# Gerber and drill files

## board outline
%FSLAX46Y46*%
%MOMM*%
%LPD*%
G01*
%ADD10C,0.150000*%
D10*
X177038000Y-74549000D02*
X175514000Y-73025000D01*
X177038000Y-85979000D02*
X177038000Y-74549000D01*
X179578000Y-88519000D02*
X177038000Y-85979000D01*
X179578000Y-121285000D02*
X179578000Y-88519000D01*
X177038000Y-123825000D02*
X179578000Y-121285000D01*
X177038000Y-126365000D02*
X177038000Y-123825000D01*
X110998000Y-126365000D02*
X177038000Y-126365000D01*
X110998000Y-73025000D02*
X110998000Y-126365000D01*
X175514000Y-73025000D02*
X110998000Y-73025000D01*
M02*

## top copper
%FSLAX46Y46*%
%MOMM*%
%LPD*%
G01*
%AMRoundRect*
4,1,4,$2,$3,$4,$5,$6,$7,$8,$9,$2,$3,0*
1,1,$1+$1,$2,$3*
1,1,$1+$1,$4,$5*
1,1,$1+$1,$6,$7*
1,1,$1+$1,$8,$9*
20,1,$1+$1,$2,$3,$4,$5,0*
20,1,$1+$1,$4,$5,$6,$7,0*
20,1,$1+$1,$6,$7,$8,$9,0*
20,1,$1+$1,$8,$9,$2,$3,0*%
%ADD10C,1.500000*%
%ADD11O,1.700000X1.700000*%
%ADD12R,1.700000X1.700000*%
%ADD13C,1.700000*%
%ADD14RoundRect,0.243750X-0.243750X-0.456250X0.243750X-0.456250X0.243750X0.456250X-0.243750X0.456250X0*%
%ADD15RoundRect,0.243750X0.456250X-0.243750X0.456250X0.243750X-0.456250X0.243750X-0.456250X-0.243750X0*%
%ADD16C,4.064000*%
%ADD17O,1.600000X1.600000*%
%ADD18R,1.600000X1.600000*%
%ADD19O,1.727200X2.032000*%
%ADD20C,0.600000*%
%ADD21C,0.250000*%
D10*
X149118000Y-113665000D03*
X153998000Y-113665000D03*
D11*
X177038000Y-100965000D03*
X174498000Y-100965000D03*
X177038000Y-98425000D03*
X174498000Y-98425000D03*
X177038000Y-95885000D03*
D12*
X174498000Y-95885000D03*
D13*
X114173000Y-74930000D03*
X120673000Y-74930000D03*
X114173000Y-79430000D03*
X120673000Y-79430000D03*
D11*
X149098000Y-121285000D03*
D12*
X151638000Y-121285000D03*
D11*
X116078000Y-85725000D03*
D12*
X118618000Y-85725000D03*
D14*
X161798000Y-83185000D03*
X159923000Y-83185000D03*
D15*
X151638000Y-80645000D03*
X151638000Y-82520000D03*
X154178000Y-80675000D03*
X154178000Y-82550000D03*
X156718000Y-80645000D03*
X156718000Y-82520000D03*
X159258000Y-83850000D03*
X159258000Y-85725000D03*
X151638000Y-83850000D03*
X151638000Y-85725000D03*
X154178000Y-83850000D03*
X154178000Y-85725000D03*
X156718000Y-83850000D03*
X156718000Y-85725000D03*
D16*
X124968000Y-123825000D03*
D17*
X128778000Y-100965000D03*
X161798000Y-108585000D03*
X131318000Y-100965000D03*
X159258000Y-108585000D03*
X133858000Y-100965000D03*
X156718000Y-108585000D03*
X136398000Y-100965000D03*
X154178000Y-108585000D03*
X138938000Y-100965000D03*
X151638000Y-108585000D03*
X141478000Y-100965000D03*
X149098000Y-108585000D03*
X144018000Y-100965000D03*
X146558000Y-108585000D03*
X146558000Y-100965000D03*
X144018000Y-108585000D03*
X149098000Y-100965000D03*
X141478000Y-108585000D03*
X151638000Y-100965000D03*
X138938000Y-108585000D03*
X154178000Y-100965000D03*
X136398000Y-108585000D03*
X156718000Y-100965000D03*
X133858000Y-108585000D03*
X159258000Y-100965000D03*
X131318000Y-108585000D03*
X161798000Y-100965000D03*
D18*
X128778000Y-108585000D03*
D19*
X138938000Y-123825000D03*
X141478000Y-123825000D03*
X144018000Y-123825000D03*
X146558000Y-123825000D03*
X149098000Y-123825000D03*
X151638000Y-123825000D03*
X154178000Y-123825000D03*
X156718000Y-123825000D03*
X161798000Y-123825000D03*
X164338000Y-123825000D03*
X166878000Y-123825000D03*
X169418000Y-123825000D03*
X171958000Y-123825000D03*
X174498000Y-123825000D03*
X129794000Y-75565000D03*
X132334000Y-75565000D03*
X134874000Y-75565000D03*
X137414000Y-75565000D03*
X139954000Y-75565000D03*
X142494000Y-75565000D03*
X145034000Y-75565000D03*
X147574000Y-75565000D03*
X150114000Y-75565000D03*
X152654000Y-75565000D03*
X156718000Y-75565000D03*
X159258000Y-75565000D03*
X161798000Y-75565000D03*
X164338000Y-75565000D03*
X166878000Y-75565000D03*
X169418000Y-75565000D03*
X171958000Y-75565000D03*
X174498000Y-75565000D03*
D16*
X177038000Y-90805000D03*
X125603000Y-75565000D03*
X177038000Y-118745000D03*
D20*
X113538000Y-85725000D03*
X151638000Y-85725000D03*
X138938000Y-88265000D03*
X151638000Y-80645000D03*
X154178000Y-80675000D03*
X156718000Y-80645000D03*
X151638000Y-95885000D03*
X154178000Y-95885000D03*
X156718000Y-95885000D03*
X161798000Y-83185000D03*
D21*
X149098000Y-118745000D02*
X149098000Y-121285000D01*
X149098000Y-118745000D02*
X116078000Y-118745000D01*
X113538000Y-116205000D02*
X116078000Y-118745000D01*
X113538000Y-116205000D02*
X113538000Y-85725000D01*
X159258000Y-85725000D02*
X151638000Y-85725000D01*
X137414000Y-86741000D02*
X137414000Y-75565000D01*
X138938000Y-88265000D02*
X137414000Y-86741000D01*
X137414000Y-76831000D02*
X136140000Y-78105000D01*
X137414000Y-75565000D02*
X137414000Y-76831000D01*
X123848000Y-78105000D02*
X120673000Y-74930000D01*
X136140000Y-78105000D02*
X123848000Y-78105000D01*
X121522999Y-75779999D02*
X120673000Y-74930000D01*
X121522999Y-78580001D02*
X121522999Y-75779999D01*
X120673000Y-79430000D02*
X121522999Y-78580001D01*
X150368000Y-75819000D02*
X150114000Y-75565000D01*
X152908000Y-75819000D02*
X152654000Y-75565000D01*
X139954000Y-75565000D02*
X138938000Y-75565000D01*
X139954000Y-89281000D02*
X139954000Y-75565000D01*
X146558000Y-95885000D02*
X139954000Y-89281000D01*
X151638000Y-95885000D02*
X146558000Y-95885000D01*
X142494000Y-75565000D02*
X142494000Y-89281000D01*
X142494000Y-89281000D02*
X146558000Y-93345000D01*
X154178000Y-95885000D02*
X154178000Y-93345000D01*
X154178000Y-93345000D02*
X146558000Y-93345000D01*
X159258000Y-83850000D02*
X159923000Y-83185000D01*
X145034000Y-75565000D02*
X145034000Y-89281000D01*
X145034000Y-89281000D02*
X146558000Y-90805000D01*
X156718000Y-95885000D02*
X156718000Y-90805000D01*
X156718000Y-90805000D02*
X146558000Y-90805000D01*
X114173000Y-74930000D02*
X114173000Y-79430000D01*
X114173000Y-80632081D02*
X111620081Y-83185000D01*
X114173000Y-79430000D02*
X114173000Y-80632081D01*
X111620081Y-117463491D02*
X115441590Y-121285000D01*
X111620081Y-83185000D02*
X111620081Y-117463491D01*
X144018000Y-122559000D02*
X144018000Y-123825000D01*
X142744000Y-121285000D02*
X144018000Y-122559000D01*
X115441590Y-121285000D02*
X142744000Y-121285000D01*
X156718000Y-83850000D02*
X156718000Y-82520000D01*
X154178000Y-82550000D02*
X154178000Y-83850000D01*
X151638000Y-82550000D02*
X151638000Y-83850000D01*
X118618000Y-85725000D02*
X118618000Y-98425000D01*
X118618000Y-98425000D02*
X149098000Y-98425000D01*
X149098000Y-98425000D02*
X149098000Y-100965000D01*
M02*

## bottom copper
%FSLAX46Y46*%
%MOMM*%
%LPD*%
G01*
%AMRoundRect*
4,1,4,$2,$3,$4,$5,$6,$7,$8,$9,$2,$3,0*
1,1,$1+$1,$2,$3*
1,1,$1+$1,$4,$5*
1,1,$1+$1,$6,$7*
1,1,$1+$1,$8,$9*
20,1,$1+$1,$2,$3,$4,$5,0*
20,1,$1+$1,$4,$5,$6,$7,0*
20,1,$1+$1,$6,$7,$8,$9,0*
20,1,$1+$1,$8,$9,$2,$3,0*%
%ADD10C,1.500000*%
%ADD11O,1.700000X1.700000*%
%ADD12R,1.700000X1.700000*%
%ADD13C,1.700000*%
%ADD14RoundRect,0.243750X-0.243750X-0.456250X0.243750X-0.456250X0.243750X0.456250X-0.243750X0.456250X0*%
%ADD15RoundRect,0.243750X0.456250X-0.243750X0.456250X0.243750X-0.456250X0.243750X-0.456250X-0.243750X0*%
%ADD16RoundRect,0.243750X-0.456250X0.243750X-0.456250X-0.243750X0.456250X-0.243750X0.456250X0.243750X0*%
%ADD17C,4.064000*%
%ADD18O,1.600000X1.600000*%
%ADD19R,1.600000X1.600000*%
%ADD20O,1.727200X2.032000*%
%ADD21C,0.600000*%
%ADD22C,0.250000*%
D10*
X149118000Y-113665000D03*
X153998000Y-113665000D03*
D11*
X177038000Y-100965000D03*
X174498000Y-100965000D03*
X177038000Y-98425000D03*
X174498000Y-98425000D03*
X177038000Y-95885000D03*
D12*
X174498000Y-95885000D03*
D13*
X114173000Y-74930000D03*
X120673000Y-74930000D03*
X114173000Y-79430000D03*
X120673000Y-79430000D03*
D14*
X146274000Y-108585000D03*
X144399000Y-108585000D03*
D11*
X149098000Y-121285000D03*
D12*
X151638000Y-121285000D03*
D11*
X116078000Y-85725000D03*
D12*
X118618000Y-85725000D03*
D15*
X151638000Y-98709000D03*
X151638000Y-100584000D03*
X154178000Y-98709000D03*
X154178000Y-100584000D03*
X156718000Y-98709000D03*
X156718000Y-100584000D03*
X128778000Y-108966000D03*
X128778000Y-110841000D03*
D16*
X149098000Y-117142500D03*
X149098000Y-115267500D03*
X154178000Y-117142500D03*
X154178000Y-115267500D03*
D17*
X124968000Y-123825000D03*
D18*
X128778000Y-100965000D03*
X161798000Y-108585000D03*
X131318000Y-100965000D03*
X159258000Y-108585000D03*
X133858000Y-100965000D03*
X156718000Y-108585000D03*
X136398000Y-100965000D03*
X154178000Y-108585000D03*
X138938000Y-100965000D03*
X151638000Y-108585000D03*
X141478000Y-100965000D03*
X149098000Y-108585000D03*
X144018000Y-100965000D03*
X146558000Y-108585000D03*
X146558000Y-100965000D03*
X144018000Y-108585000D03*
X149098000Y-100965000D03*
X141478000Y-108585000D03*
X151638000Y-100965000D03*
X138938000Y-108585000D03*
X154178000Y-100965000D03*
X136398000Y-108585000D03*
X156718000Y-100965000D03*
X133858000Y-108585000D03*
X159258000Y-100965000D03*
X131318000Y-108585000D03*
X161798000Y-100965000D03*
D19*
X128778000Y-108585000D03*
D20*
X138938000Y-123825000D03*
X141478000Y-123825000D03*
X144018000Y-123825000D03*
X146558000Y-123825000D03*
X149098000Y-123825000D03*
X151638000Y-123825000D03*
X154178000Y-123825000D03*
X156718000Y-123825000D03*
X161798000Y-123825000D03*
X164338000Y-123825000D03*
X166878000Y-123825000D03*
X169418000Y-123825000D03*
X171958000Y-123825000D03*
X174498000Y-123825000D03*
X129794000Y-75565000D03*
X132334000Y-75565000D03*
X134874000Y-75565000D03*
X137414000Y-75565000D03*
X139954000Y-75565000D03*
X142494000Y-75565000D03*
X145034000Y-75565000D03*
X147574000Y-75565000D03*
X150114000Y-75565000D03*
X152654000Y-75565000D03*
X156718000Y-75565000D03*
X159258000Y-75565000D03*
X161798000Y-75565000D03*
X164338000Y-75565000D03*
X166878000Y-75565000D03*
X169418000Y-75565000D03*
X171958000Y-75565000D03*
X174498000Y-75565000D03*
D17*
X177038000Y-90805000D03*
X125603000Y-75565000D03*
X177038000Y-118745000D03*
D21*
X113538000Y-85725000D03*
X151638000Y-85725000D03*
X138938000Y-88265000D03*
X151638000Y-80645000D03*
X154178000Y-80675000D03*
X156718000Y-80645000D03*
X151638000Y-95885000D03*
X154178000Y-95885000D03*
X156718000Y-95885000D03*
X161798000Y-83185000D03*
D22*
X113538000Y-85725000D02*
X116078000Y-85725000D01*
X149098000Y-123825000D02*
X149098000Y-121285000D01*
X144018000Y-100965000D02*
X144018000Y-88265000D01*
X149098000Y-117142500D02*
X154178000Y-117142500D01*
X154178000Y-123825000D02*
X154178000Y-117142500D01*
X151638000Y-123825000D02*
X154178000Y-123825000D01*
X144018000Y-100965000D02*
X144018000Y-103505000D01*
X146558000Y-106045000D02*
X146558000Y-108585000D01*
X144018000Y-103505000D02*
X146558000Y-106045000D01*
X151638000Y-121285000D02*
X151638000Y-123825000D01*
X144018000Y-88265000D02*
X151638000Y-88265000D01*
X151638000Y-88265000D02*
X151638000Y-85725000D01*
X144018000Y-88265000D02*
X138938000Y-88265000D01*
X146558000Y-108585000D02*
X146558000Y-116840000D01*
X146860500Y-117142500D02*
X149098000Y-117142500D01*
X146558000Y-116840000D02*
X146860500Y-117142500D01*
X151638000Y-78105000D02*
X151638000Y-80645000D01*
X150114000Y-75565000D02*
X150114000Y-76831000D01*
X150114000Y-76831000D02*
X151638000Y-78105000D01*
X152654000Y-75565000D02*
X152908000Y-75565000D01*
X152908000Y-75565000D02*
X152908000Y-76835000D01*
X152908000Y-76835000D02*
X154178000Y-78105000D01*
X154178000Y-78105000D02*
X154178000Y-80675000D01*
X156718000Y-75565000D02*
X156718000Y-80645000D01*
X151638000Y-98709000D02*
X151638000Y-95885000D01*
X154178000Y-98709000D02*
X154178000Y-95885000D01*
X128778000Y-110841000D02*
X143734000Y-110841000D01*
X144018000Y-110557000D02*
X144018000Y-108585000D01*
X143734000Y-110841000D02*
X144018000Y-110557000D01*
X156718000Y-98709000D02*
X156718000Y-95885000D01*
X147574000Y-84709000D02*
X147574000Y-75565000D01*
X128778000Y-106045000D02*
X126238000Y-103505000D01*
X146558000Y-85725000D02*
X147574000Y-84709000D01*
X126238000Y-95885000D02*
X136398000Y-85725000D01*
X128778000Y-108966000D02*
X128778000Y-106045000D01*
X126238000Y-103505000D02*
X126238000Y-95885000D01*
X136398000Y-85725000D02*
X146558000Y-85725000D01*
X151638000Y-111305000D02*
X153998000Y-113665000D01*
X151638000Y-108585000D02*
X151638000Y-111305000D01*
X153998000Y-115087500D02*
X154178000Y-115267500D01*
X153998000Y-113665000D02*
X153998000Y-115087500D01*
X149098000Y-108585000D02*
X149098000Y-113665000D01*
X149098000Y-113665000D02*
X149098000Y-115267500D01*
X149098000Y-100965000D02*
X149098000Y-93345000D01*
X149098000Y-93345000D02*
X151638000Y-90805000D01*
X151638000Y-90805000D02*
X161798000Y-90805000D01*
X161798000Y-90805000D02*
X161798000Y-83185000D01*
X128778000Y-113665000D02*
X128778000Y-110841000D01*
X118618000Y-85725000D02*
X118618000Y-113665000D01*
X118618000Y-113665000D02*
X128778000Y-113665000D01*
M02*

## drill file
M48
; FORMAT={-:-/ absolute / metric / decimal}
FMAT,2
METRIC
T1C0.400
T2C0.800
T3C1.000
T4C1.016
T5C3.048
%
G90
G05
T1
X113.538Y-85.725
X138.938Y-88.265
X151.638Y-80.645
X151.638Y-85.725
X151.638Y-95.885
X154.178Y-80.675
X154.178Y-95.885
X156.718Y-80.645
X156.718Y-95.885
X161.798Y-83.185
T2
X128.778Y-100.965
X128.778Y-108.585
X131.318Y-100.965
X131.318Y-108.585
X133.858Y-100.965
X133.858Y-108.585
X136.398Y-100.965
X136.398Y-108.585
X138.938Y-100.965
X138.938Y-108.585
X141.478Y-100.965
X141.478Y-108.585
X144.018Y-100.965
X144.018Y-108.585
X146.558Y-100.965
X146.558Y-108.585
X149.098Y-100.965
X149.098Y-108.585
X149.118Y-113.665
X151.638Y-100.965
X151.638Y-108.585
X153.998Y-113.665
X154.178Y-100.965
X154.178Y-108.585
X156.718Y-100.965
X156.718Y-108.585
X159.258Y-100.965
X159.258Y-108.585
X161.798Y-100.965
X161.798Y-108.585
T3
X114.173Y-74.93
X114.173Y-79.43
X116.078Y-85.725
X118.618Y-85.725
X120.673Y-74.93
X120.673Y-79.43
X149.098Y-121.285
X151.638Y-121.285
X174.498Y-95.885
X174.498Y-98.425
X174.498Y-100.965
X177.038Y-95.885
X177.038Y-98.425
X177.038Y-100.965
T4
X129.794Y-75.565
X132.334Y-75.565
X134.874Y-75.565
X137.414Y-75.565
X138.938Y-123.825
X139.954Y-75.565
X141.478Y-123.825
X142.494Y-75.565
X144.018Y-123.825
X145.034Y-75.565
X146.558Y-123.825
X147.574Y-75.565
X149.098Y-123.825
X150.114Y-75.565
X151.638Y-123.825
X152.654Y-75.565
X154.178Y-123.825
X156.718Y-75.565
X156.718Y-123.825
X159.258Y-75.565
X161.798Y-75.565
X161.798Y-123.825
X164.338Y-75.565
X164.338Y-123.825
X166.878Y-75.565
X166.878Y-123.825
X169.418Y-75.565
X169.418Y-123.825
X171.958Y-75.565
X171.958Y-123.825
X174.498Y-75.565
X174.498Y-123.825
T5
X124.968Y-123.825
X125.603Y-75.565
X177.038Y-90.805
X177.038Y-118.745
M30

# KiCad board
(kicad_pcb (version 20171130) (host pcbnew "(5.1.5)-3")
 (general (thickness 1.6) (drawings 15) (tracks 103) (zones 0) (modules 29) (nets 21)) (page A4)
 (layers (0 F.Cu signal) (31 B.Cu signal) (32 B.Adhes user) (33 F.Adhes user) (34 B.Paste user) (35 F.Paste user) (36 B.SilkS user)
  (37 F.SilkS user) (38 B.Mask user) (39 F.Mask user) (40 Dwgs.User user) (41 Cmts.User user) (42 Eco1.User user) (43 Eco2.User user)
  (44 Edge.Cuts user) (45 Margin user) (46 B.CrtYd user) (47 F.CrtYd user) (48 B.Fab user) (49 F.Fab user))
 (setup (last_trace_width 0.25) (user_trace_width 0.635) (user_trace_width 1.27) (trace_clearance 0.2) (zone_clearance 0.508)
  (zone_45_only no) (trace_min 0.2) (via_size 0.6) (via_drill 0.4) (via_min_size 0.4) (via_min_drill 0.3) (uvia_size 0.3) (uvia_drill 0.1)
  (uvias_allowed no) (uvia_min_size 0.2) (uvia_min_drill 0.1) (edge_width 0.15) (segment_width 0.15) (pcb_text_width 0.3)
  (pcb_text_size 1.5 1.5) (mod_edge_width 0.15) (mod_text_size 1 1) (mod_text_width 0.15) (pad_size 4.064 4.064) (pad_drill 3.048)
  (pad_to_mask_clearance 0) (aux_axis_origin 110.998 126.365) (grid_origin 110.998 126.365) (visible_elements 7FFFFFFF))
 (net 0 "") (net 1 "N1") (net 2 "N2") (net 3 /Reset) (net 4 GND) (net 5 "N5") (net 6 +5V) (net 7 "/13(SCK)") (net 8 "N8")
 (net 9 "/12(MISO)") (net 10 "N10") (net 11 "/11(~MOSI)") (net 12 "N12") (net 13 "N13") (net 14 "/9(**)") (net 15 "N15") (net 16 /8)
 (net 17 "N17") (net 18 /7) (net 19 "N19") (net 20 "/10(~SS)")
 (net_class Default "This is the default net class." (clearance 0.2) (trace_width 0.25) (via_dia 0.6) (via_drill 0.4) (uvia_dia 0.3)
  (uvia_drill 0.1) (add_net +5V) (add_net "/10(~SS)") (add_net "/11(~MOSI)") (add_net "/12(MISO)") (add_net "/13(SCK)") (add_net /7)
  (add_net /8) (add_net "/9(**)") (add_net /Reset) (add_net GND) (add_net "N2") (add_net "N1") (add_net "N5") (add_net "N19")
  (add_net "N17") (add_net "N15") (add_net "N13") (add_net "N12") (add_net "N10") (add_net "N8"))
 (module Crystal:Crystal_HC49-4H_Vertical (layer F.Cu) (at 153.998 113.665 180)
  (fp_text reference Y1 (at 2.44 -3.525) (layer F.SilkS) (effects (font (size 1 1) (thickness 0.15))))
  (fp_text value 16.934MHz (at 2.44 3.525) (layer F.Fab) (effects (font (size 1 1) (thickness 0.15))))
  (pad 2 thru_hole circle (at 4.88 0 180) (size 1.5 1.5) (drill 0.8) (layers *.Cu *.Mask) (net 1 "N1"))
  (pad 1 thru_hole circle (at 0 0 180) (size 1.5 1.5) (drill 0.8) (layers *.Cu *.Mask) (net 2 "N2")))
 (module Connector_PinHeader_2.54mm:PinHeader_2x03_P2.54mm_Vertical (layer F.Cu) (at 174.498 95.885)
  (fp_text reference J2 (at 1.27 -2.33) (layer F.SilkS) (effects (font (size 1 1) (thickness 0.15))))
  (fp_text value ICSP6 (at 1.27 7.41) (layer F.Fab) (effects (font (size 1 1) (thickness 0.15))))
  (pad 6 thru_hole oval (at 2.54 5.08) (size 1.7 1.7) (drill 1) (layers *.Cu *.Mask))
  (pad 5 thru_hole oval (at 0 5.08) (size 1.7 1.7) (drill 1) (layers *.Cu *.Mask))
  (pad 4 thru_hole oval (at 2.54 2.54) (size 1.7 1.7) (drill 1) (layers *.Cu *.Mask))
  (pad 3 thru_hole oval (at 0 2.54) (size 1.7 1.7) (drill 1) (layers *.Cu *.Mask))
  (pad 2 thru_hole oval (at 2.54 0) (size 1.7 1.7) (drill 1) (layers *.Cu *.Mask))
  (pad 1 thru_hole rect (at 0 0) (size 1.7 1.7) (drill 1) (layers *.Cu *.Mask)))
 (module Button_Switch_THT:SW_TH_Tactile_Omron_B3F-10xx (layer F.Cu) (at 114.173 74.93)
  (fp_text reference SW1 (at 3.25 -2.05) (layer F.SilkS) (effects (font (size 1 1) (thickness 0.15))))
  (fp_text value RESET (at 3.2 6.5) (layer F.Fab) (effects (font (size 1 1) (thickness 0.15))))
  (pad 1 thru_hole circle (at 0 0) (size 1.7 1.7) (drill 1) (layers *.Cu *.Mask) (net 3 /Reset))
  (pad 2 thru_hole circle (at 6.5 0) (size 1.7 1.7) (drill 1) (layers *.Cu *.Mask) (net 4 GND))
  (pad 3 thru_hole circle (at 0 4.5) (size 1.7 1.7) (drill 1) (layers *.Cu *.Mask) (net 3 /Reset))
  (pad 4 thru_hole circle (at 6.5 4.5) (size 1.7 1.7) (drill 1) (layers *.Cu *.Mask) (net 4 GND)))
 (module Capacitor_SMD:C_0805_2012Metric (layer B.Cu) (at 145.3365 108.585)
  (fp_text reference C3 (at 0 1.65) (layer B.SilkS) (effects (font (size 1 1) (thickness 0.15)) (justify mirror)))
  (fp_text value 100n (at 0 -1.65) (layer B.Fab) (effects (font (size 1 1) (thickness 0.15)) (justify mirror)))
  (pad 2 smd roundrect (at 0.9375 0) (size 0.975 1.4) (layers B.Cu B.Paste B.Mask) (roundrect_rratio 0.25) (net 4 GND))
  (pad 1 smd roundrect (at -0.9375 0) (size 0.975 1.4) (layers B.Cu B.Paste B.Mask) (roundrect_rratio 0.25) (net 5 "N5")))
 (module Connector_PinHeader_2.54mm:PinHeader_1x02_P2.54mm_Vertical (layer F.Cu) (at 151.638 121.285 270)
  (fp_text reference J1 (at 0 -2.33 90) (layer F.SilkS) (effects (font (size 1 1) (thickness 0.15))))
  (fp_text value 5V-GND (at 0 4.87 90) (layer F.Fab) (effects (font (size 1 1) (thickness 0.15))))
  (pad 2 thru_hole oval (at 0 2.54 270) (size 1.7 1.7) (drill 1) (layers *.Cu *.Mask) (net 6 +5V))
  (pad 1 thru_hole rect (at 0 0 270) (size 1.7 1.7) (drill 1) (layers *.Cu *.Mask) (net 4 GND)))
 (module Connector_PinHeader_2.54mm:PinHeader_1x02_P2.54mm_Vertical (layer F.Cu) (at 118.618 85.725 270)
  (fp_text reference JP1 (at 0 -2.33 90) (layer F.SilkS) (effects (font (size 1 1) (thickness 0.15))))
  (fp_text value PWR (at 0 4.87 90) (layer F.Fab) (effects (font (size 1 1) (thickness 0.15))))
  (pad 2 thru_hole oval (at 0 2.54 270) (size 1.7 1.7) (drill 1) (layers *.Cu *.Mask) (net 6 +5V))
  (pad 1 thru_hole rect (at 0 0 270) (size 1.7 1.7) (drill 1) (layers *.Cu *.Mask) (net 5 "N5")))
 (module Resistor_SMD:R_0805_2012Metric (layer B.Cu) (at 151.638 99.6465 90)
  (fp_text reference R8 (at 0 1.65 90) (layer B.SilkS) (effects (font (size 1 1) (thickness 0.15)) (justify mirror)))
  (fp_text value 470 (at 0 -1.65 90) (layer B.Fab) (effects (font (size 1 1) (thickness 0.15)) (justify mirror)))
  (pad 2 smd roundrect (at 0.9375 0 90) (size 0.975 1.4) (layers B.Cu B.Paste B.Mask) (roundrect_rratio 0.25) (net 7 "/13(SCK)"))
  (pad 1 smd roundrect (at -0.9375 0 90) (size 0.975 1.4) (layers B.Cu B.Paste B.Mask) (roundrect_rratio 0.25) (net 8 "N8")))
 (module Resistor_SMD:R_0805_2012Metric (layer B.Cu) (at 154.178 99.6465 90)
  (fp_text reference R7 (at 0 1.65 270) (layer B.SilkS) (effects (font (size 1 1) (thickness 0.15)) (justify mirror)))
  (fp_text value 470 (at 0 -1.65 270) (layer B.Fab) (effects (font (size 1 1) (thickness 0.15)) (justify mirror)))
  (pad 2 smd roundrect (at 0.9375 0 90) (size 0.975 1.4) (layers B.Cu B.Paste B.Mask) (roundrect_rratio 0.25) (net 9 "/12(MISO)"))
  (pad 1 smd roundrect (at -0.9375 0 90) (size 0.975 1.4) (layers B.Cu B.Paste B.Mask) (roundrect_rratio 0.25) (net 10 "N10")))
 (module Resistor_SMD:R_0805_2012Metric (layer B.Cu) (at 156.718 99.6465 90)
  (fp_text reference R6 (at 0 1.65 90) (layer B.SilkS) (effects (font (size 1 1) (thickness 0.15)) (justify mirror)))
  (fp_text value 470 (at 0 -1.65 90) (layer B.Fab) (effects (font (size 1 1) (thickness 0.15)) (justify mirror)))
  (pad 2 smd roundrect (at 0.9375 0 90) (size 0.975 1.4) (layers B.Cu B.Paste B.Mask) (roundrect_rratio 0.25) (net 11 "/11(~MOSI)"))
  (pad 1 smd roundrect (at -0.9375 0 90) (size 0.975 1.4) (layers B.Cu B.Paste B.Mask) (roundrect_rratio 0.25) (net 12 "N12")))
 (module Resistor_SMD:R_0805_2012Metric (layer F.Cu) (at 160.8605 83.185)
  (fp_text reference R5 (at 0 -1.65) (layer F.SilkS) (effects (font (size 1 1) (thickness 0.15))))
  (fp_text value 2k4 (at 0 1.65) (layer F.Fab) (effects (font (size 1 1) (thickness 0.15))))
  (pad 2 smd roundrect (at 0.9375 0) (size 0.975 1.4) (layers F.Cu F.Paste F.Mask) (roundrect_rratio 0.25) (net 5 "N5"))
  (pad 1 smd roundrect (at -0.9375 0) (size 0.975 1.4) (layers F.Cu F.Paste F.Mask) (roundrect_rratio 0.25) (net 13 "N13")))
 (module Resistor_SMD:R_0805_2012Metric (layer F.Cu) (at 151.638 81.5825 90)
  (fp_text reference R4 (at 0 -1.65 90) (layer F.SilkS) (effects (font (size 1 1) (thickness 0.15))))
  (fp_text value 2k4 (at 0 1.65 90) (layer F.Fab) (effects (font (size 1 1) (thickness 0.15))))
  (pad 2 smd roundrect (at 0.9375 0 90) (size 0.975 1.4) (layers F.Cu F.Paste F.Mask) (roundrect_rratio 0.25) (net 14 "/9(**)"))
  (pad 1 smd roundrect (at -0.9375 0 90) (size 0.975 1.4) (layers F.Cu F.Paste F.Mask) (roundrect_rratio 0.25) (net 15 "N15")))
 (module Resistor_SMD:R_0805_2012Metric (layer F.Cu) (at 154.178 81.6125 90)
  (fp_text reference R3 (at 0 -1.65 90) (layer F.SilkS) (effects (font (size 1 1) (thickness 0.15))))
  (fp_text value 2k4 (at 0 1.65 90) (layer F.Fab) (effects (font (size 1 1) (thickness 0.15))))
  (pad 2 smd roundrect (at 0.9375 0 90) (size 0.975 1.4) (layers F.Cu F.Paste F.Mask) (roundrect_rratio 0.25) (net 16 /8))
  (pad 1 smd roundrect (at -0.9375 0 90) (size 0.975 1.4) (layers F.Cu F.Paste F.Mask) (roundrect_rratio 0.25) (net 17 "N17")))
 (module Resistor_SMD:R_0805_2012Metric (layer F.Cu) (at 156.718 81.5825 90)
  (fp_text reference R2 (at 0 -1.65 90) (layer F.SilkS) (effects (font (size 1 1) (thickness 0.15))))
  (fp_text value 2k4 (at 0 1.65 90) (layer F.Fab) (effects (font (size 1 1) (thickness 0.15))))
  (pad 2 smd roundrect (at 0.9375 0 90) (size 0.975 1.4) (layers F.Cu F.Paste F.Mask) (roundrect_rratio 0.25) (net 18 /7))
  (pad 1 smd roundrect (at -0.9375 0 90) (size 0.975 1.4) (layers F.Cu F.Paste F.Mask) (roundrect_rratio 0.25) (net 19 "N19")))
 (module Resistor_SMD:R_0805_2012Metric (layer B.Cu) (at 128.778 109.9035 90)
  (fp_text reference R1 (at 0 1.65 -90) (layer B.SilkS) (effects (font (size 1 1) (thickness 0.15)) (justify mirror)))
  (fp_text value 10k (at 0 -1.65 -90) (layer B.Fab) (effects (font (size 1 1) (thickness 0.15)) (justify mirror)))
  (pad 2 smd roundrect (at 0.9375 0 90) (size 0.975 1.4) (layers B.Cu B.Paste B.Mask) (roundrect_rratio 0.25) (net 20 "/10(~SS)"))
  (pad 1 smd roundrect (at -0.9375 0 90) (size 0.975 1.4) (layers B.Cu B.Paste B.Mask) (roundrect_rratio 0.25) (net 5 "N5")))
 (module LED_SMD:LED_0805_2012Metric (layer F.Cu) (at 159.258 84.7875 90)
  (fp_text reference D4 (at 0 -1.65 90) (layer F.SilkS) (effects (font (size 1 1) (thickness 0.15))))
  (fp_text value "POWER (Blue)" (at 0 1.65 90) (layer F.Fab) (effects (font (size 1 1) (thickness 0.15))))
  (pad 2 smd roundrect (at 0.9375 0 90) (size 0.975 1.4) (layers F.Cu F.Paste F.Mask) (roundrect_rratio 0.25) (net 13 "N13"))
  (pad 1 smd roundrect (at -0.9375 0 90) (size 0.975 1.4) (layers F.Cu F.Paste F.Mask) (roundrect_rratio 0.25) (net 4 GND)))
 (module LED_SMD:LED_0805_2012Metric (layer F.Cu) (at 151.638 84.7875 90)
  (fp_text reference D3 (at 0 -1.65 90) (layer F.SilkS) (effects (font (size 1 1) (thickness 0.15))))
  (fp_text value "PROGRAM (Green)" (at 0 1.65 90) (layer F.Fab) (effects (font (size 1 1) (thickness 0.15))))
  (pad 2 smd roundrect (at 0.9375 0 90) (size 0.975 1.4) (layers F.Cu F.Paste F.Mask) (roundrect_rratio 0.25) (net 15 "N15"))
  (pad 1 smd roundrect (at -0.9375 0 90) (size 0.975 1.4) (layers F.Cu F.Paste F.Mask) (roundrect_rratio 0.25) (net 4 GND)))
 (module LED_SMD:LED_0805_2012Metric (layer F.Cu) (at 154.178 84.7875 90)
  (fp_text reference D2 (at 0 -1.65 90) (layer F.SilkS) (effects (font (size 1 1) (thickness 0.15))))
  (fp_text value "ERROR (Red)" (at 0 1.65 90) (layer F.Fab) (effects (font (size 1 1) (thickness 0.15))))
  (pad 2 smd roundrect (at 0.9375 0 90) (size 0.975 1.4) (layers F.Cu F.Paste F.Mask) (roundrect_rratio 0.25) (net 17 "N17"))
  (pad 1 smd roundrect (at -0.9375 0 90) (size 0.975 1.4) (layers F.Cu F.Paste F.Mask) (roundrect_rratio 0.25) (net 4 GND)))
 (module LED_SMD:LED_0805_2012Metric (layer F.Cu) (at 156.718 84.7875 90)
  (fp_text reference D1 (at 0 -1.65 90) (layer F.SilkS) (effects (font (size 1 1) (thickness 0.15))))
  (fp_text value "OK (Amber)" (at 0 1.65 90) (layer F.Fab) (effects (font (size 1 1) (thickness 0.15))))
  (pad 2 smd roundrect (at 0.9375 0 90) (size 0.975 1.4) (layers F.Cu F.Paste F.Mask) (roundrect_rratio 0.25) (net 19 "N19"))
  (pad 1 smd roundrect (at -0.9375 0 90) (size 0.975 1.4) (layers F.Cu F.Paste F.Mask) (roundrect_rratio 0.25) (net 4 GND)))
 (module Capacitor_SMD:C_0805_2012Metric (layer B.Cu) (at 149.098 116.205 270)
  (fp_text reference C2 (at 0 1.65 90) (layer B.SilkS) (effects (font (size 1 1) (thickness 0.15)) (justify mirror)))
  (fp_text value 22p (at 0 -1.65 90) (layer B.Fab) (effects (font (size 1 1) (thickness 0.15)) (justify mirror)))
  (pad 2 smd roundrect (at 0.9375 0 270) (size 0.975 1.4) (layers B.Cu B.Paste B.Mask) (roundrect_rratio 0.25) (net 4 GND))
  (pad 1 smd roundrect (at -0.9375 0 270) (size 0.975 1.4) (layers B.Cu B.Paste B.Mask) (roundrect_rratio 0.25) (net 1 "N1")))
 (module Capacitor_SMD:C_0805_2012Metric (layer B.Cu) (at 154.178 116.205 270)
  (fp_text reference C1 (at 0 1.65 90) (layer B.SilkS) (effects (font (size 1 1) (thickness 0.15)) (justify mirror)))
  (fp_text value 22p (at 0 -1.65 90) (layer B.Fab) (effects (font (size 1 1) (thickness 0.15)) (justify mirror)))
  (pad 2 smd roundrect (at 0.9375 0 270) (size 0.975 1.4) (layers B.Cu B.Paste B.Mask) (roundrect_rratio 0.25) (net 4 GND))
  (pad 1 smd roundrect (at -0.9375 0 270) (size 0.975 1.4) (layers B.Cu B.Paste B.Mask) (roundrect_rratio 0.25) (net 2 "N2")))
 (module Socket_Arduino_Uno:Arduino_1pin (layer F.Cu) (at 124.968 123.825 90)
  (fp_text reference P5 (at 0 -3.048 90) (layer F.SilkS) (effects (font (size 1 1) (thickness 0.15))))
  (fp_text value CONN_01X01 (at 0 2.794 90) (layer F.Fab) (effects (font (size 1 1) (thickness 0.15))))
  (pad 1 thru_hole circle (at 0 0 90) (size 4.064 4.064) (drill 3.048) (layers *.Cu *.Mask F.SilkS)))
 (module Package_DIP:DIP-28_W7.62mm (layer F.Cu) (at 128.778 108.585 90)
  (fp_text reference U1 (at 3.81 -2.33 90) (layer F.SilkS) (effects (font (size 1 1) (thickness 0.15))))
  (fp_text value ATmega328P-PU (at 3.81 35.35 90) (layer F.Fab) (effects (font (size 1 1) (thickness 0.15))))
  (pad 28 thru_hole oval (at 7.62 0 90) (size 1.6 1.6) (drill 0.8) (layers *.Cu *.Mask))
  (pad 14 thru_hole oval (at 0 33.02 90) (size 1.6 1.6) (drill 0.8) (layers *.Cu *.Mask))
  (pad 27 thru_hole oval (at 7.62 2.54 90) (size 1.6 1.6) (drill 0.8) (layers *.Cu *.Mask))
  (pad 13 thru_hole oval (at 0 30.48 90) (size 1.6 1.6) (drill 0.8) (layers *.Cu *.Mask))
  (pad 26 thru_hole oval (at 7.62 5.08 90) (size 1.6 1.6) (drill 0.8) (layers *.Cu *.Mask))
  (pad 12 thru_hole oval (at 0 27.94 90) (size 1.6 1.6) (drill 0.8) (layers *.Cu *.Mask))
  (pad 25 thru_hole oval (at 7.62 7.62 90) (size 1.6 1.6) (drill 0.8) (layers *.Cu *.Mask))
  (pad 11 thru_hole oval (at 0 25.4 90) (size 1.6 1.6) (drill 0.8) (layers *.Cu *.Mask))
  (pad 24 thru_hole oval (at 7.62 10.16 90) (size 1.6 1.6) (drill 0.8) (layers *.Cu *.Mask))
  (pad 10 thru_hole oval (at 0 22.86 90) (size 1.6 1.6) (drill 0.8) (layers *.Cu *.Mask) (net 2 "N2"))
  (pad 23 thru_hole oval (at 7.62 12.7 90) (size 1.6 1.6) (drill 0.8) (layers *.Cu *.Mask))
  (pad 9 thru_hole oval (at 0 20.32 90) (size 1.6 1.6) (drill 0.8) (layers *.Cu *.Mask) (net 1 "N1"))
  (pad 22 thru_hole oval (at 7.62 15.24 90) (size 1.6 1.6) (drill 0.8) (layers *.Cu *.Mask) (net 4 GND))
  (pad 8 thru_hole oval (at 0 17.78 90) (size 1.6 1.6) (drill 0.8) (layers *.Cu *.Mask) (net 4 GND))
  (pad 21 thru_hole oval (at 7.62 17.78 90) (size 1.6 1.6) (drill 0.8) (layers *.Cu *.Mask))
  (pad 7 thru_hole oval (at 0 15.24 90) (size 1.6 1.6) (drill 0.8) (layers *.Cu *.Mask) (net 5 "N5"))
  (pad 20 thru_hole oval (at 7.62 20.32 90) (size 1.6 1.6) (drill 0.8) (layers *.Cu *.Mask) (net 5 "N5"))
  (pad 6 thru_hole oval (at 0 12.7 90) (size 1.6 1.6) (drill 0.8) (layers *.Cu *.Mask))
  (pad 19 thru_hole oval (at 7.62 22.86 90) (size 1.6 1.6) (drill 0.8) (layers *.Cu *.Mask) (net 8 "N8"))
  (pad 5 thru_hole oval (at 0 10.16 90) (size 1.6 1.6) (drill 0.8) (layers *.Cu *.Mask))
  (pad 18 thru_hole oval (at 7.62 25.4 90) (size 1.6 1.6) (drill 0.8) (layers *.Cu *.Mask) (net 10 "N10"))
  (pad 4 thru_hole oval (at 0 7.62 90) (size 1.6 1.6) (drill 0.8) (layers *.Cu *.Mask))
  (pad 17 thru_hole oval (at 7.62 27.94 90) (size 1.6 1.6) (drill 0.8) (layers *.Cu *.Mask) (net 12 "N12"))
  (pad 3 thru_hole oval (at 0 5.08 90) (size 1.6 1.6) (drill 0.8) (layers *.Cu *.Mask))
  (pad 16 thru_hole oval (at 7.62 30.48 90) (size 1.6 1.6) (drill 0.8) (layers *.Cu *.Mask))
  (pad 2 thru_hole oval (at 0 2.54 90) (size 1.6 1.6) (drill 0.8) (layers *.Cu *.Mask))
  (pad 15 thru_hole oval (at 7.62 33.02 90) (size 1.6 1.6) (drill 0.8) (layers *.Cu *.Mask))
  (pad 1 thru_hole rect (at 0 0 90) (size 1.6 1.6) (drill 0.8) (layers *.Cu *.Mask) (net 20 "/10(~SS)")))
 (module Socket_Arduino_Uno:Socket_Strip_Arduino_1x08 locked (layer F.Cu) (at 138.938 123.825)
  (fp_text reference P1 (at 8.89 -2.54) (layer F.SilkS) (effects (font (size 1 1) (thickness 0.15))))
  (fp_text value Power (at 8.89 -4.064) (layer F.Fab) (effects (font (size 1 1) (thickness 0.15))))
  (pad 1 thru_hole oval (at 0 0) (size 1.7272 2.032) (drill 1.016) (layers *.Cu *.Mask F.SilkS))
  (pad 2 thru_hole oval (at 2.54 0) (size 1.7272 2.032) (drill 1.016) (layers *.Cu *.Mask F.SilkS))
  (pad 3 thru_hole oval (at 5.08 0) (size 1.7272 2.032) (drill 1.016) (layers *.Cu *.Mask F.SilkS) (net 3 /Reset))
  (pad 4 thru_hole oval (at 7.62 0) (size 1.7272 2.032) (drill 1.016) (layers *.Cu *.Mask F.SilkS))
  (pad 5 thru_hole oval (at 10.16 0) (size 1.7272 2.032) (drill 1.016) (layers *.Cu *.Mask F.SilkS) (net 6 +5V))
  (pad 6 thru_hole oval (at 12.7 0) (size 1.7272 2.032) (drill 1.016) (layers *.Cu *.Mask F.SilkS) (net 4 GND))
  (pad 7 thru_hole oval (at 15.24 0) (size 1.7272 2.032) (drill 1.016) (layers *.Cu *.Mask F.SilkS) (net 4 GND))
  (pad 8 thru_hole oval (at 17.78 0) (size 1.7272 2.032) (drill 1.016) (layers *.Cu *.Mask F.SilkS)))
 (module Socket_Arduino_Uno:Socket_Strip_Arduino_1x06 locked (layer F.Cu) (at 161.798 123.825)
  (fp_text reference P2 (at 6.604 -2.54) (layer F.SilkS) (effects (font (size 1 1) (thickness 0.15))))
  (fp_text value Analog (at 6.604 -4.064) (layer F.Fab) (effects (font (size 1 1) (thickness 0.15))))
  (pad 1 thru_hole oval (at 0 0) (size 1.7272 2.032) (drill 1.016) (layers *.Cu *.Mask F.SilkS))
  (pad 2 thru_hole oval (at 2.54 0) (size 1.7272 2.032) (drill 1.016) (layers *.Cu *.Mask F.SilkS))
  (pad 3 thru_hole oval (at 5.08 0) (size 1.7272 2.032) (drill 1.016) (layers *.Cu *.Mask F.SilkS))
  (pad 4 thru_hole oval (at 7.62 0) (size 1.7272 2.032) (drill 1.016) (layers *.Cu *.Mask F.SilkS))
  (pad 5 thru_hole oval (at 10.16 0) (size 1.7272 2.032) (drill 1.016) (layers *.Cu *.Mask F.SilkS))
  (pad 6 thru_hole oval (at 12.7 0) (size 1.7272 2.032) (drill 1.016) (layers *.Cu *.Mask F.SilkS)))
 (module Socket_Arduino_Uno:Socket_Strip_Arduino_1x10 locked (layer F.Cu) (at 129.794 75.565)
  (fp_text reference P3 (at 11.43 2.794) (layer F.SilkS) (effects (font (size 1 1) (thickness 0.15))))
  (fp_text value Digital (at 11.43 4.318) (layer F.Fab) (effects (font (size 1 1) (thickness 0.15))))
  (pad 1 thru_hole oval (at 0 0) (size 1.7272 2.032) (drill 1.016) (layers *.Cu *.Mask F.SilkS))
  (pad 2 thru_hole oval (at 2.54 0) (size 1.7272 2.032) (drill 1.016) (layers *.Cu *.Mask F.SilkS))
  (pad 3 thru_hole oval (at 5.08 0) (size 1.7272 2.032) (drill 1.016) (layers *.Cu *.Mask F.SilkS))
  (pad 4 thru_hole oval (at 7.62 0) (size 1.7272 2.032) (drill 1.016) (layers *.Cu *.Mask F.SilkS) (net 4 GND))
  (pad 5 thru_hole oval (at 10.16 0) (size 1.7272 2.032) (drill 1.016) (layers *.Cu *.Mask F.SilkS) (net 7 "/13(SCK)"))
  (pad 6 thru_hole oval (at 12.7 0) (size 1.7272 2.032) (drill 1.016) (layers *.Cu *.Mask F.SilkS) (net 9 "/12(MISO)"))
  (pad 7 thru_hole oval (at 15.24 0) (size 1.7272 2.032) (drill 1.016) (layers *.Cu *.Mask F.SilkS) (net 11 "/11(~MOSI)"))
  (pad 8 thru_hole oval (at 17.78 0) (size 1.7272 2.032) (drill 1.016) (layers *.Cu *.Mask F.SilkS) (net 20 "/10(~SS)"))
  (pad 9 thru_hole oval (at 20.32 0) (size 1.7272 2.032) (drill 1.016) (layers *.Cu *.Mask F.SilkS) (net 14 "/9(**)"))
  (pad 10 thru_hole oval (at 22.86 0) (size 1.7272 2.032) (drill 1.016) (layers *.Cu *.Mask F.SilkS) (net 16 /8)))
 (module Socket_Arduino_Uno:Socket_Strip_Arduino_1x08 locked (layer F.Cu) (at 156.718 75.565)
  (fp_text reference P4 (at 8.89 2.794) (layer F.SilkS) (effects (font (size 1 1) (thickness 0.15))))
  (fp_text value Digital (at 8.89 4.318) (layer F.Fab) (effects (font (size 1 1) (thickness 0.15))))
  (pad 1 thru_hole oval (at 0 0) (size 1.7272 2.032) (drill 1.016) (layers *.Cu *.Mask F.SilkS) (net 18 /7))
  (pad 2 thru_hole oval (at 2.54 0) (size 1.7272 2.032) (drill 1.016) (layers *.Cu *.Mask F.SilkS))
  (pad 3 thru_hole oval (at 5.08 0) (size 1.7272 2.032) (drill 1.016) (layers *.Cu *.Mask F.SilkS))
  (pad 4 thru_hole oval (at 7.62 0) (size 1.7272 2.032) (drill 1.016) (layers *.Cu *.Mask F.SilkS))
  (pad 5 thru_hole oval (at 10.16 0) (size 1.7272 2.032) (drill 1.016) (layers *.Cu *.Mask F.SilkS))
  (pad 6 thru_hole oval (at 12.7 0) (size 1.7272 2.032) (drill 1.016) (layers *.Cu *.Mask F.SilkS))
  (pad 7 thru_hole oval (at 15.24 0) (size 1.7272 2.032) (drill 1.016) (layers *.Cu *.Mask F.SilkS))
  (pad 8 thru_hole oval (at 17.78 0) (size 1.7272 2.032) (drill 1.016) (layers *.Cu *.Mask F.SilkS)))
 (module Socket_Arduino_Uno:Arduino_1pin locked (layer F.Cu) (at 177.038 90.805 90)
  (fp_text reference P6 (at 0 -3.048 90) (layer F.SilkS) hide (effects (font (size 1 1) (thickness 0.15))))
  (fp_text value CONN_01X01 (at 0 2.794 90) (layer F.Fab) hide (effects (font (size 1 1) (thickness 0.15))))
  (pad 1 thru_hole circle (at 0 0 90) (size 4.064 4.064) (drill 3.048) (layers *.Cu *.Mask F.SilkS)))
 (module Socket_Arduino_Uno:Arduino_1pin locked (layer F.Cu) (at 125.603 75.565 90)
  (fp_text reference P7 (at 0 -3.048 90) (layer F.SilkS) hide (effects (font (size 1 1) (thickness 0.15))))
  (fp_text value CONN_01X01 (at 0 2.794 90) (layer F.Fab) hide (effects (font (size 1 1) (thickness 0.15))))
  (pad 1 thru_hole circle (at 0 0 90) (size 4.064 4.064) (drill 3.048) (layers *.Cu *.Mask F.SilkS)))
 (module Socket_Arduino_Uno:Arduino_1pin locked (layer F.Cu) (at 177.038 118.745 90)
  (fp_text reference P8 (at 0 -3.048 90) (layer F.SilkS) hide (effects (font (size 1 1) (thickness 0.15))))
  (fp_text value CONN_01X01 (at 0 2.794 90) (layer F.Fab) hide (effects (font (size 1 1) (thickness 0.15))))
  (pad 1 thru_hole circle (at 0 0 90) (size 4.064 4.064) (drill 3.048) (layers *.Cu *.Mask F.SilkS)))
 (gr_line (start 177.038 74.549) (end 175.514 73.025) (angle 90) (layer Edge.Cuts) (width 0.15))
 (gr_line (start 177.038 85.979) (end 177.038 74.549) (angle 90) (layer Edge.Cuts) (width 0.15))
 (gr_line (start 179.578 88.519) (end 177.038 85.979) (angle 90) (layer Edge.Cuts) (width 0.15))
 (gr_line (start 179.578 121.285) (end 179.578 88.519) (angle 90) (layer Edge.Cuts) (width 0.15))
 (gr_line (start 177.038 123.825) (end 179.578 121.285) (angle 90) (layer Edge.Cuts) (width 0.15))
 (gr_line (start 177.038 126.365) (end 177.038 123.825) (angle 90) (layer Edge.Cuts) (width 0.15))
 (gr_line (start 110.998 126.365) (end 177.038 126.365) (angle 90) (layer Edge.Cuts) (width 0.15))
 (gr_line (start 110.998 73.025) (end 110.998 126.365) (angle 90) (layer Edge.Cuts) (width 0.15))
 (gr_line (start 175.514 73.025) (end 110.998 73.025) (angle 90) (layer Edge.Cuts) (width 0.15))
 (via (at 113.538 85.725) (size 0.6) (drill 0.4) (layers F.Cu B.Cu) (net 6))
 (segment (start 113.538 85.725) (end 116.078 85.725) (width 0.25) (layer B.Cu) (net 6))
 (segment (start 149.098 123.825) (end 149.098 121.285) (width 0.25) (layer B.Cu) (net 6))
 (segment (start 149.098 118.745) (end 149.098 121.285) (width 0.25) (layer F.Cu) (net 6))
 (segment (start 149.098 118.745) (end 116.078 118.745) (width 0.25) (layer F.Cu) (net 6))
 (segment (start 113.538 116.205) (end 116.078 118.745) (width 0.25) (layer F.Cu) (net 6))
 (segment (start 113.538 116.205) (end 113.538 85.725) (width 0.25) (layer F.Cu) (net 6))
 (segment (start 144.018 100.965) (end 144.018 88.265) (width 0.25) (layer B.Cu) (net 4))
 (segment (start 149.098 117.1425) (end 154.178 117.1425) (width 0.25) (layer B.Cu) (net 4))
 (segment (start 154.178 123.825) (end 154.178 117.1425) (width 0.25) (layer B.Cu) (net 4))
 (segment (start 151.638 123.825) (end 154.178 123.825) (width 0.25) (layer B.Cu) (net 4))
 (segment (start 144.018 100.965) (end 144.018 103.505) (width 0.25) (layer B.Cu) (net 4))
 (segment (start 146.558 106.045) (end 146.558 108.585) (width 0.25) (layer B.Cu) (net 4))
 (segment (start 144.018 103.505) (end 146.558 106.045) (width 0.25) (layer B.Cu) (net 4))
 (segment (start 151.638 121.285) (end 151.638 123.825) (width 0.25) (layer B.Cu) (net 4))
 (segment (start 159.258 85.725) (end 151.638 85.725) (width 0.25) (layer F.Cu) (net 4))
 (segment (start 144.018 88.265) (end 151.638 88.265) (width 0.25) (layer B.Cu) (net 4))
 (segment (start 151.638 88.265) (end 151.638 85.725) (width 0.25) (layer B.Cu) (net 4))
 (via (at 151.638 85.725) (size 0.6) (drill 0.4) (layers F.Cu B.Cu) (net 4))
 (segment (start 144.018 88.265) (end 138.938 88.265) (width 0.25) (layer B.Cu) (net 4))
 (via (at 138.938 88.265) (size 0.6) (drill 0.4) (layers F.Cu B.Cu) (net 4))
 (segment (start 137.414 86.741) (end 137.414 75.565) (width 0.25) (layer F.Cu) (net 4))
 (segment (start 138.938 88.265) (end 137.414 86.741) (width 0.25) (layer F.Cu) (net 4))
 (segment (start 146.558 108.585) (end 146.558 116.84) (width 0.25) (layer B.Cu) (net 4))
 (segment (start 146.8605 117.1425) (end 149.098 117.1425) (width 0.25) (layer B.Cu) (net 4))
 (segment (start 146.558 116.84) (end 146.8605 117.1425) (width 0.25) (layer B.Cu) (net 4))
 (segment (start 137.414 76.831) (end 136.14 78.105) (width 0.25) (layer F.Cu) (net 4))
 (segment (start 137.414 75.565) (end 137.414 76.831) (width 0.25) (layer F.Cu) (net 4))
 (segment (start 123.848 78.105) (end 120.673 74.93) (width 0.25) (layer F.Cu) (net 4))
 (segment (start 136.14 78.105) (end 123.848 78.105) (width 0.25) (layer F.Cu) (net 4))
 (segment (start 121.522999 75.779999) (end 120.673 74.93) (width 0.25) (layer F.Cu) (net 4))
 (segment (start 121.522999 78.580001) (end 121.522999 75.779999) (width 0.25) (layer F.Cu) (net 4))
 (segment (start 120.673 79.43) (end 121.522999 78.580001) (width 0.25) (layer F.Cu) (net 4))
 (segment (start 150.368 75.819) (end 150.114 75.565) (width 0.25) (layer F.Cu) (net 14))
 (via (at 151.638 80.645) (size 0.6) (drill 0.4) (layers F.Cu B.Cu) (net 14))
 (segment (start 151.638 78.105) (end 151.638 80.645) (width 0.25) (layer B.Cu) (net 14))
 (segment (start 150.114 75.565) (end 150.114 76.831) (width 0.25) (layer B.Cu) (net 14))
 (segment (start 150.114 76.831) (end 151.638 78.105) (width 0.25) (layer B.Cu) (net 14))
 (segment (start 152.908 75.819) (end 152.654 75.565) (width 0.25) (layer F.Cu) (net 16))
 (segment (start 152.654 75.565) (end 152.908 75.565) (width 0.25) (layer B.Cu) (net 16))
 (segment (start 152.908 75.565) (end 152.908 76.835) (width 0.25) (layer B.Cu) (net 16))
 (segment (start 152.908 76.835) (end 154.178 78.105) (width 0.25) (layer B.Cu) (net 16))
 (via (at 154.178 80.675) (size 0.6) (drill 0.4) (layers F.Cu B.Cu) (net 16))
 (segment (start 154.178 78.105) (end 154.178 80.675) (width 0.25) (layer B.Cu) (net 16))
 (segment (start 156.718 75.565) (end 156.718 80.645) (width 0.25) (layer B.Cu) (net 18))
 (via (at 156.718 80.645) (size 0.6) (drill 0.4) (layers F.Cu B.Cu) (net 18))
 (segment (start 139.954 75.565) (end 138.938 75.565) (width 0.25) (layer F.Cu) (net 7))
 (segment (start 139.954 89.281) (end 139.954 75.565) (width 0.25) (layer F.Cu) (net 7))
 (segment (start 146.558 95.885) (end 139.954 89.281) (width 0.25) (layer F.Cu) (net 7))
 (segment (start 151.638 98.709) (end 151.638 95.885) (width 0.25) (layer B.Cu) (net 7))
 (via (at 151.638 95.885) (size 0.6) (drill 0.4) (layers F.Cu B.Cu) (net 7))
 (segment (start 151.638 95.885) (end 146.558 95.885) (width 0.25) (layer F.Cu) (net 7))
 (segment (start 142.494 75.565) (end 142.494 89.281) (width 0.25) (layer F.Cu) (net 9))
 (segment (start 142.494 89.281) (end 146.558 93.345) (width 0.25) (layer F.Cu) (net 9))
 (segment (start 154.178 98.709) (end 154.178 95.885) (width 0.25) (layer B.Cu) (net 9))
 (via (at 154.178 95.885) (size 0.6) (drill 0.4) (layers F.Cu B.Cu) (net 9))
 (segment (start 154.178 95.885) (end 154.178 93.345) (width 0.25) (layer F.Cu) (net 9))
 (segment (start 154.178 93.345) (end 146.558 93.345) (width 0.25) (layer F.Cu) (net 9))
 (segment (start 159.258 83.85) (end 159.923 83.185) (width 0.25) (layer F.Cu) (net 13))
 (segment (start 128.778 110.841) (end 143.734 110.841) (width 0.25) (layer B.Cu) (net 5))
 (segment (start 144.018 110.557) (end 144.018 108.585) (width 0.25) (layer B.Cu) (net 5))
 (segment (start 143.734 110.841) (end 144.018 110.557) (width 0.25) (layer B.Cu) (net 5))
 (segment (start 145.034 75.565) (end 145.034 89.281) (width 0.25) (layer F.Cu) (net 11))
 (segment (start 145.034 89.281) (end 146.558 90.805) (width 0.25) (layer F.Cu) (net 11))
 (segment (start 156.718 98.709) (end 156.718 95.885) (width 0.25) (layer B.Cu) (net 11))
 (via (at 156.718 95.885) (size 0.6) (drill 0.4) (layers F.Cu B.Cu) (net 11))
 (segment (start 156.718 95.885) (end 156.718 90.805) (width 0.25) (layer F.Cu) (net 11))
 (segment (start 156.718 90.805) (end 146.558 90.805) (width 0.25) (layer F.Cu) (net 11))
 (segment (start 147.574 84.709) (end 147.574 75.565) (width 0.25) (layer B.Cu) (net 20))
 (segment (start 128.778 106.045) (end 126.238 103.505) (width 0.25) (layer B.Cu) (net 20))
 (segment (start 146.558 85.725) (end 147.574 84.709) (width 0.25) (layer B.Cu) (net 20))
 (segment (start 126.238 95.885) (end 136.398 85.725) (width 0.25) (layer B.Cu) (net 20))
 (segment (start 128.778 108.966) (end 128.778 106.045) (width 0.25) (layer B.Cu) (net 20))
 (segment (start 126.238 103.505) (end 126.238 95.885) (width 0.25) (layer B.Cu) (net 20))
 (segment (start 136.398 85.725) (end 146.558 85.725) (width 0.25) (layer B.Cu) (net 20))
 (segment (start 151.638 111.305) (end 153.998 113.665) (width 0.25) (layer B.Cu) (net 2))
 (segment (start 151.638 108.585) (end 151.638 111.305) (width 0.25) (layer B.Cu) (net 2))
 (segment (start 153.998 115.0875) (end 154.178 115.2675) (width 0.25) (layer B.Cu) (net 2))
 (segment (start 153.998 113.665) (end 153.998 115.0875) (width 0.25) (layer B.Cu) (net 2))
 (segment (start 149.098 108.585) (end 149.098 113.665) (width 0.25) (layer B.Cu) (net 1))
 (segment (start 149.098 113.665) (end 149.098 115.2675) (width 0.25) (layer B.Cu) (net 1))
 (segment (start 114.173 74.93) (end 114.173 79.43) (width 0.25) (layer F.Cu) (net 3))
 (segment (start 114.173 80.632081) (end 111.620081 83.185) (width 0.25) (layer F.Cu) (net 3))
 (segment (start 114.173 79.43) (end 114.173 80.632081) (width 0.25) (layer F.Cu) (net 3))
 (segment (start 111.620081 117.463491) (end 115.44159 121.285) (width 0.25) (layer F.Cu) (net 3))
 (segment (start 111.620081 83.185) (end 111.620081 117.463491) (width 0.25) (layer F.Cu) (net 3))
 (segment (start 144.018 122.559) (end 144.018 123.825) (width 0.25) (layer F.Cu) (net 3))
 (segment (start 142.744 121.285) (end 144.018 122.559) (width 0.25) (layer F.Cu) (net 3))
 (segment (start 115.44159 121.285) (end 142.744 121.285) (width 0.25) (layer F.Cu) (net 3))
 (segment (start 156.718 83.85) (end 156.718 82.52) (width 0.25) (layer F.Cu) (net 19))
 (segment (start 154.178 82.55) (end 154.178 83.85) (width 0.25) (layer F.Cu) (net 17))
 (segment (start 151.638 82.55) (end 151.638 83.85) (width 0.25) (layer F.Cu) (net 15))
 (segment (start 118.618 85.725) (end 118.618 98.425) (width 0.25) (layer F.Cu) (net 5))
 (segment (start 118.618 98.425) (end 149.098 98.425) (width 0.25) (layer F.Cu) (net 5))
 (segment (start 149.098 98.425) (end 149.098 100.965) (width 0.25) (layer F.Cu) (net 5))
 (segment (start 149.098 100.965) (end 149.098 93.345) (width 0.25) (layer B.Cu) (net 5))
 (segment (start 149.098 93.345) (end 151.638 90.805) (width 0.25) (layer B.Cu) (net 5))
 (segment (start 151.638 90.805) (end 161.798 90.805) (width 0.25) (layer B.Cu) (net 5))
 (segment (start 161.798 90.805) (end 161.798 83.185) (width 0.25) (layer B.Cu) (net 5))
 (via (at 161.798 83.185) (size 0.6) (drill 0.4) (layers F.Cu B.Cu) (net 5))
 (segment (start 128.778 113.665) (end 128.778 110.841) (width 0.25) (layer B.Cu) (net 5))
 (segment (start 118.618 85.725) (end 118.618 113.665) (width 0.25) (layer B.Cu) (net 5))
 (segment (start 118.618 113.665) (end 128.778 113.665) (width 0.25) (layer B.Cu) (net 5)))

